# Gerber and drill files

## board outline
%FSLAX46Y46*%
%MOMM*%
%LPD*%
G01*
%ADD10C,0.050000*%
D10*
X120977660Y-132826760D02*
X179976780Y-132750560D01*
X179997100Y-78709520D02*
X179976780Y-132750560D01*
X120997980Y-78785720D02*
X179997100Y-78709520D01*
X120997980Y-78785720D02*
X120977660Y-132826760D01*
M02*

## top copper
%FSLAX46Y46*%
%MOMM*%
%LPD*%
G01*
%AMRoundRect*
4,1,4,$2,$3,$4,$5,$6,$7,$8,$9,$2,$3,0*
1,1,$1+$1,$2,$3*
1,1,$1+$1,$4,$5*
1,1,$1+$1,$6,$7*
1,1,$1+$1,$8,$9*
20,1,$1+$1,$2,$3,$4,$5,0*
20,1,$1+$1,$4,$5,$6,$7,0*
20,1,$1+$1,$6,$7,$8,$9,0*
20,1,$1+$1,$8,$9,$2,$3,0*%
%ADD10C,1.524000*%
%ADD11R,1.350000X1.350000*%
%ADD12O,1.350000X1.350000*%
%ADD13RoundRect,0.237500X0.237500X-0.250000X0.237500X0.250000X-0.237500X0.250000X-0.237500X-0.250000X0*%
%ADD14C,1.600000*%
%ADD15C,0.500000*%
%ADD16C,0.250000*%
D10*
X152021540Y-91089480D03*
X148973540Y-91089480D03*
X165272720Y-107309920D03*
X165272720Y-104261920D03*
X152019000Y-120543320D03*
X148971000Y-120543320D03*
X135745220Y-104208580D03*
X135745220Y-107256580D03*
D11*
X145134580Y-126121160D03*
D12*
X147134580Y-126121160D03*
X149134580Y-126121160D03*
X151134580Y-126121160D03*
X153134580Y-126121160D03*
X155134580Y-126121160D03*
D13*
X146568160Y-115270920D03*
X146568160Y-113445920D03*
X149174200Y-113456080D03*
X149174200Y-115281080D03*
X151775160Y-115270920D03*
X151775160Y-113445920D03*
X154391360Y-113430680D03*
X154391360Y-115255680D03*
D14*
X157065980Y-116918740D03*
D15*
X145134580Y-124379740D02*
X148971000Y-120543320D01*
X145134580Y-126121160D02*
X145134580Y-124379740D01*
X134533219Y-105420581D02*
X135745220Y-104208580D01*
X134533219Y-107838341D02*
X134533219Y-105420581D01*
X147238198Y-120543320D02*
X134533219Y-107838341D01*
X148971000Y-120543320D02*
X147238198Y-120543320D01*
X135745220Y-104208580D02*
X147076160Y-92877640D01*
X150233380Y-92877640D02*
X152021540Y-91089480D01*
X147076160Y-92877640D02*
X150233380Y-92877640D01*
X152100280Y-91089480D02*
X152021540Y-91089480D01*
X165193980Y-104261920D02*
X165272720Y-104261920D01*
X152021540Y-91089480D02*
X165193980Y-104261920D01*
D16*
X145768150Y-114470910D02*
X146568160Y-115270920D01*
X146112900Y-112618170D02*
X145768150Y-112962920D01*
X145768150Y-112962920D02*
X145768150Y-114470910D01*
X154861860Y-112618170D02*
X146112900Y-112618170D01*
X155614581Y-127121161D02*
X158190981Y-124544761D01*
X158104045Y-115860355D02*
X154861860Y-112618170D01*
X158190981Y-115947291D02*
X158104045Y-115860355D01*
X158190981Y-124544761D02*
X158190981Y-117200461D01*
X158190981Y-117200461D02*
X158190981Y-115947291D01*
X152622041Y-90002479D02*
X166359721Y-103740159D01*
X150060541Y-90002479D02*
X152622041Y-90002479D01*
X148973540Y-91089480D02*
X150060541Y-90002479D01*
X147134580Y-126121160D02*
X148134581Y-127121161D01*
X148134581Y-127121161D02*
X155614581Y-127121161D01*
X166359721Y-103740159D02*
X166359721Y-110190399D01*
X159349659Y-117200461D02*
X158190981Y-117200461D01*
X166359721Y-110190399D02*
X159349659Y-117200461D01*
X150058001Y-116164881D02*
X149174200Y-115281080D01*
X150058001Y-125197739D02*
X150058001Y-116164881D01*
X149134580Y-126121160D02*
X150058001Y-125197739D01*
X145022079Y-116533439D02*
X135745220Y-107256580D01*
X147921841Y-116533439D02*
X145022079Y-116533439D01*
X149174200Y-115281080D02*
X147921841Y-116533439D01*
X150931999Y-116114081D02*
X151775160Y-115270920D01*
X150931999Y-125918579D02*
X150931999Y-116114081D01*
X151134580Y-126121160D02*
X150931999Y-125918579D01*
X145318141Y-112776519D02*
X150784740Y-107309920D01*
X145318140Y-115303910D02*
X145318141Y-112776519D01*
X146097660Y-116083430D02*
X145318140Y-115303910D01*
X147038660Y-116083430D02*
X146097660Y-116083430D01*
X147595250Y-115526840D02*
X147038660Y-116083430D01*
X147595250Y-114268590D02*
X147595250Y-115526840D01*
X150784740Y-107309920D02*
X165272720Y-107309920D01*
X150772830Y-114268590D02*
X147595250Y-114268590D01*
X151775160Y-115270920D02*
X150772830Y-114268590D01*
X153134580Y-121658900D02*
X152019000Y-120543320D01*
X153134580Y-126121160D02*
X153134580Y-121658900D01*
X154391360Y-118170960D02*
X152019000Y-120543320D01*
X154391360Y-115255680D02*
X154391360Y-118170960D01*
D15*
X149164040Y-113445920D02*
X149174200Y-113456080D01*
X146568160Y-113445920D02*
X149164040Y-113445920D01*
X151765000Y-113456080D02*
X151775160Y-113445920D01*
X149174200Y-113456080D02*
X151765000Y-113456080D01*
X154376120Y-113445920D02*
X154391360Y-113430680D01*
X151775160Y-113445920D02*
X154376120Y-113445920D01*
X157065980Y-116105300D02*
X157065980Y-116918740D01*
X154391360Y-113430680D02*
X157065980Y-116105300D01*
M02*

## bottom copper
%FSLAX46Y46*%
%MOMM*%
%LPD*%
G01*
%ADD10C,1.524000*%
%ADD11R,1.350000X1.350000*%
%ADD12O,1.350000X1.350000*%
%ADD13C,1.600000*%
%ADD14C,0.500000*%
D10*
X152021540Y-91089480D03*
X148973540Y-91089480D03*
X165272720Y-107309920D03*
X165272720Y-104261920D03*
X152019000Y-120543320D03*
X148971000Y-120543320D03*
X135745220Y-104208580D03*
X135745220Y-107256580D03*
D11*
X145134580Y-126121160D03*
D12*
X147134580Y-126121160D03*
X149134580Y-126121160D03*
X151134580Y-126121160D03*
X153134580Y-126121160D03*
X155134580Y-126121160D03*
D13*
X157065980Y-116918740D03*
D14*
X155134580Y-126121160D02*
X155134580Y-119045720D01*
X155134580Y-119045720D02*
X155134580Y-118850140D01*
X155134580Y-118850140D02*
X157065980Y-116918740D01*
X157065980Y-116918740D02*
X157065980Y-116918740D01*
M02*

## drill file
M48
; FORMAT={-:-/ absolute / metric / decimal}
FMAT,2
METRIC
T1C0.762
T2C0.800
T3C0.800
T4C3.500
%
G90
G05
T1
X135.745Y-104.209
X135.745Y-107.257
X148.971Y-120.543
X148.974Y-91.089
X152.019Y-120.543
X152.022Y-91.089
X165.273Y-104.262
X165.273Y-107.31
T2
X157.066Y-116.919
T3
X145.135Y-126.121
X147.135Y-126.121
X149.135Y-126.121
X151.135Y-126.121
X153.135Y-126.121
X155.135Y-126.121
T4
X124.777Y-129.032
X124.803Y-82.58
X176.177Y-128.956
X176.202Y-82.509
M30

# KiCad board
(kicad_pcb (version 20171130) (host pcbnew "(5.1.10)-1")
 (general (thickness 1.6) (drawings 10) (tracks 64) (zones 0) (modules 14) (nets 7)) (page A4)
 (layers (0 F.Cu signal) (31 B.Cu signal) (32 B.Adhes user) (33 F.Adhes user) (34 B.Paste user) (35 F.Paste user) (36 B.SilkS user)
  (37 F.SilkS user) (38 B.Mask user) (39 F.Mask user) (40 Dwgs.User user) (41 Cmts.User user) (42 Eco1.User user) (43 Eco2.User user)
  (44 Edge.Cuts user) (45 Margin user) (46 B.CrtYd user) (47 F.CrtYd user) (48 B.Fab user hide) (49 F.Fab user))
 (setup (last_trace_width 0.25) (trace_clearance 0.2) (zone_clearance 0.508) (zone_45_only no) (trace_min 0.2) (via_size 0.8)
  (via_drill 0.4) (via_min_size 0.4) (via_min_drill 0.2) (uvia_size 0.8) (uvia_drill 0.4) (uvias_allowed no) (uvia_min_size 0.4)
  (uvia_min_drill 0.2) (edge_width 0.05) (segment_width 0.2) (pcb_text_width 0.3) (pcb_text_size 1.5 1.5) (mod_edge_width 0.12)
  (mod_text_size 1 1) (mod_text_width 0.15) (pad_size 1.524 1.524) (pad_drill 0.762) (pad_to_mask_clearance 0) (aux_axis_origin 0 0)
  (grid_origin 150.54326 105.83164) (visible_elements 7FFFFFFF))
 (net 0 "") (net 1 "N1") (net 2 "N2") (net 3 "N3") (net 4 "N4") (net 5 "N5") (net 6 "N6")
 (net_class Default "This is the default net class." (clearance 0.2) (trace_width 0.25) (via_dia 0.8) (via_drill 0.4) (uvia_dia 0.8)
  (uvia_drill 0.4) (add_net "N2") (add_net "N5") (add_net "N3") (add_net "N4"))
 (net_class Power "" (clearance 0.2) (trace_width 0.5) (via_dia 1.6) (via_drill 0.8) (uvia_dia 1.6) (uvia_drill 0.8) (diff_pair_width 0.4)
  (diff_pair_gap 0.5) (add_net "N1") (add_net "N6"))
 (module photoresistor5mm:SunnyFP (layer B.Cu) (at 150.43912 105.8418)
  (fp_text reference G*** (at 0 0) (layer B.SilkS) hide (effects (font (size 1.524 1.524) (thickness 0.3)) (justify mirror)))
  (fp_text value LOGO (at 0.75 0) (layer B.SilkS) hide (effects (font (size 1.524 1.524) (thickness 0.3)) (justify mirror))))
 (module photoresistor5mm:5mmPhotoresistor (layer F.Cu) (at 150.49754 91.08948 180)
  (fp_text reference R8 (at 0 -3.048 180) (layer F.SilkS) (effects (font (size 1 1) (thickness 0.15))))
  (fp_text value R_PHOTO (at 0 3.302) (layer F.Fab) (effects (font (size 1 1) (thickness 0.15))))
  (pad 1 thru_hole circle (at -1.524 0 180) (size 1.524 1.524) (drill 0.762) (layers *.Cu *.Mask) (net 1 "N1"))
  (pad 2 thru_hole circle (at 1.524 0 180) (size 1.524 1.524) (drill 0.762) (layers *.Cu *.Mask) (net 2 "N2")))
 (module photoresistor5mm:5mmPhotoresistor (layer F.Cu) (at 165.27272 105.78592 270)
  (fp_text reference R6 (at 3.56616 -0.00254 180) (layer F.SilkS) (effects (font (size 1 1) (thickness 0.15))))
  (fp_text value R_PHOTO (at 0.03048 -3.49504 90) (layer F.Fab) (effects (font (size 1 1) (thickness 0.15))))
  (pad 2 thru_hole circle (at 1.524 0 270) (size 1.524 1.524) (drill 0.762) (layers *.Cu *.Mask) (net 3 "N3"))
  (pad 1 thru_hole circle (at -1.524 0 270) (size 1.524 1.524) (drill 0.762) (layers *.Cu *.Mask) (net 1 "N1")))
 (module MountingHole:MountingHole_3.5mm (layer F.Cu) (at 176.17694 128.9558)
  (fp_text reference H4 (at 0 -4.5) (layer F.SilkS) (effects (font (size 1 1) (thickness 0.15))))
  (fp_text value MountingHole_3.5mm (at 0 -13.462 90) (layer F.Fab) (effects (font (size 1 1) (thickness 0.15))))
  (pad 1 np_thru_hole circle (at 0 0) (size 3.5 3.5) (drill 3.5) (layers *.Cu *.Mask)))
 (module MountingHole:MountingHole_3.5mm (layer F.Cu) (at 124.7775 129.032)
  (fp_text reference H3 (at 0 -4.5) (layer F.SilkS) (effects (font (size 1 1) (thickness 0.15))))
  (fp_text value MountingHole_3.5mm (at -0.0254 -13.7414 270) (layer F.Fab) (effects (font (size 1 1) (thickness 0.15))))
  (pad 1 np_thru_hole circle (at 0 0) (size 3.5 3.5) (drill 3.5) (layers *.Cu *.Mask)))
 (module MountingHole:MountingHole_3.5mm (layer F.Cu) (at 176.20234 82.50936 180)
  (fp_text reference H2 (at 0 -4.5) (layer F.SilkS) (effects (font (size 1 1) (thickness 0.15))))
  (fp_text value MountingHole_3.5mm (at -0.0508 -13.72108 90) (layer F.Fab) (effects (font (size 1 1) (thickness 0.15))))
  (pad 1 np_thru_hole circle (at 0 0 180) (size 3.5 3.5) (drill 3.5) (layers *.Cu *.Mask)))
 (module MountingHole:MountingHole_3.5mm (layer F.Cu) (at 124.8029 82.58048 180)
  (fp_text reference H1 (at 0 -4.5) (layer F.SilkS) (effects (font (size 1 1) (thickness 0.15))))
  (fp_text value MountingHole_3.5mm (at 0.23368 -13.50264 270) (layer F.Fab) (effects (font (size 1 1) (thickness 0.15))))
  (pad 1 np_thru_hole circle (at 0 0 180) (size 3.5 3.5) (drill 3.5) (layers *.Cu *.Mask)))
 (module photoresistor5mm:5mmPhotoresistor (layer F.Cu) (at 150.495 120.54332)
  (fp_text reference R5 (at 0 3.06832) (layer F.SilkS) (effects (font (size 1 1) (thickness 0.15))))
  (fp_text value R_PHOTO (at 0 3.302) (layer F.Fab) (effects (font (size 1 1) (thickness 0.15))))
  (pad 2 thru_hole circle (at 1.524 0) (size 1.524 1.524) (drill 0.762) (layers *.Cu *.Mask) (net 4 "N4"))
  (pad 1 thru_hole circle (at -1.524 0) (size 1.524 1.524) (drill 0.762) (layers *.Cu *.Mask) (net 1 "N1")))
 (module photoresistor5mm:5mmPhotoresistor (layer F.Cu) (at 135.74522 105.73258 270)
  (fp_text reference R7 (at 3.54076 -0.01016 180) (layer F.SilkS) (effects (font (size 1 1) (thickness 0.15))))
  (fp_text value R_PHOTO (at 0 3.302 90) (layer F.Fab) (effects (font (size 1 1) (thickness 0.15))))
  (pad 1 thru_hole circle (at -1.524 0 270) (size 1.524 1.524) (drill 0.762) (layers *.Cu *.Mask) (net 1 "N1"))
  (pad 2 thru_hole circle (at 1.524 0 270) (size 1.524 1.524) (drill 0.762) (layers *.Cu *.Mask) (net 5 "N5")))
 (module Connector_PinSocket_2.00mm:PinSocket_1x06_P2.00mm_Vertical (layer B.Cu) (at 145.13458 126.12116 270)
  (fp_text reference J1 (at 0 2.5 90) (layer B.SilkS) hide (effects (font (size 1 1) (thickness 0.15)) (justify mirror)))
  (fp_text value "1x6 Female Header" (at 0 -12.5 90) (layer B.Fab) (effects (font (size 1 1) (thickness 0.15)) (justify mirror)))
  (pad 1 thru_hole rect (at 0 0 270) (size 1.35 1.35) (drill 0.8) (layers *.Cu *.Mask) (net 1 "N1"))
  (pad 2 thru_hole oval (at 0 -2 270) (size 1.35 1.35) (drill 0.8) (layers *.Cu *.Mask) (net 2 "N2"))
  (pad 3 thru_hole oval (at 0 -4 270) (size 1.35 1.35) (drill 0.8) (layers *.Cu *.Mask) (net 5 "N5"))
  (pad 4 thru_hole oval (at 0 -6 270) (size 1.35 1.35) (drill 0.8) (layers *.Cu *.Mask) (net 3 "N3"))
  (pad 5 thru_hole oval (at 0 -8 270) (size 1.35 1.35) (drill 0.8) (layers *.Cu *.Mask) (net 4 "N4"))
  (pad 6 thru_hole oval (at 0 -10 270) (size 1.35 1.35) (drill 0.8) (layers *.Cu *.Mask) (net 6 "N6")))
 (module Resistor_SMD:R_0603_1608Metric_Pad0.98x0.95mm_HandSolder (layer F.Cu) (at 146.56816 114.35842 90)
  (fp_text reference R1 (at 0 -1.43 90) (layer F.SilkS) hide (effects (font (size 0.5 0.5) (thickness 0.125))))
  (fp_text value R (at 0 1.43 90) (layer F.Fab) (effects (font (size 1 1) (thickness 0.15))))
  (pad 1 smd roundrect (at -0.9125 0 90) (size 0.975 0.95) (layers F.Cu F.Paste F.Mask) (roundrect_rratio 0.25) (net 2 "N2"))
  (pad 2 smd roundrect (at 0.9125 0 90) (size 0.975 0.95) (layers F.Cu F.Paste F.Mask) (roundrect_rratio 0.25) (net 6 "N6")))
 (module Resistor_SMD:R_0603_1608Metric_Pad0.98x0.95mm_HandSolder (layer F.Cu) (at 149.1742 114.36858 90)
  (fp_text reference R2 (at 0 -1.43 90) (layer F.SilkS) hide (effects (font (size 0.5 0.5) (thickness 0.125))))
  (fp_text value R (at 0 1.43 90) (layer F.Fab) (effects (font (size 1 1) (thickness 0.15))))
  (pad 2 smd roundrect (at 0.9125 0 90) (size 0.975 0.95) (layers F.Cu F.Paste F.Mask) (roundrect_rratio 0.25) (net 6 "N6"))
  (pad 1 smd roundrect (at -0.9125 0 90) (size 0.975 0.95) (layers F.Cu F.Paste F.Mask) (roundrect_rratio 0.25) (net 5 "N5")))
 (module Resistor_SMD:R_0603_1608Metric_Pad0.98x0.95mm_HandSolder (layer F.Cu) (at 151.77516 114.35842 90)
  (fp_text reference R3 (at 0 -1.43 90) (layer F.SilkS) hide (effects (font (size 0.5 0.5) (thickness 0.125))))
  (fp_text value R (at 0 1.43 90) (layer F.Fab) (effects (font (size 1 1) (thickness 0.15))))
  (pad 1 smd roundrect (at -0.9125 0 90) (size 0.975 0.95) (layers F.Cu F.Paste F.Mask) (roundrect_rratio 0.25) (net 3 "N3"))
  (pad 2 smd roundrect (at 0.9125 0 90) (size 0.975 0.95) (layers F.Cu F.Paste F.Mask) (roundrect_rratio 0.25) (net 6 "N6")))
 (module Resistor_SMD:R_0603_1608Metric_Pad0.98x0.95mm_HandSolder (layer F.Cu) (at 154.39136 114.34318 90)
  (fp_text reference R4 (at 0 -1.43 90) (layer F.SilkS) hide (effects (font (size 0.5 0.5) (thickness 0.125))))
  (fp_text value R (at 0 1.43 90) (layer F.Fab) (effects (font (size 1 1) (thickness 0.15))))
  (pad 2 smd roundrect (at 0.9125 0 90) (size 0.975 0.95) (layers F.Cu F.Paste F.Mask) (roundrect_rratio 0.25) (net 6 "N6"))
  (pad 1 smd roundrect (at -0.9125 0 90) (size 0.975 0.95) (layers F.Cu F.Paste F.Mask) (roundrect_rratio 0.25) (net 4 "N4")))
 (gr_line (start 120.97766 132.82676) (end 179.97678 132.75056) (layer Edge.Cuts) (width 0.05))
 (gr_line (start 179.9971 78.70952) (end 179.97678 132.75056) (layer Edge.Cuts) (width 0.05))
 (gr_line (start 120.99798 78.78572) (end 179.9971 78.70952) (layer Edge.Cuts) (width 0.05))
 (gr_line (start 120.99798 78.78572) (end 120.97766 132.82676) (layer Edge.Cuts) (width 0.05))
 (segment (start 145.13458 124.37974) (end 148.971 120.54332) (width 0.5) (layer F.Cu) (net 1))
 (segment (start 145.13458 126.12116) (end 145.13458 124.37974) (width 0.5) (layer F.Cu) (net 1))
 (segment (start 134.533219 105.420581) (end 135.74522 104.20858) (width 0.5) (layer F.Cu) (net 1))
 (segment (start 134.533219 107.838341) (end 134.533219 105.420581) (width 0.5) (layer F.Cu) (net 1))
 (segment (start 147.238198 120.54332) (end 134.533219 107.838341) (width 0.5) (layer F.Cu) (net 1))
 (segment (start 148.971 120.54332) (end 147.238198 120.54332) (width 0.5) (layer F.Cu) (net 1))
 (segment (start 135.74522 104.20858) (end 147.07616 92.87764) (width 0.5) (layer F.Cu) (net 1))
 (segment (start 150.23338 92.87764) (end 152.02154 91.08948) (width 0.5) (layer F.Cu) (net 1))
 (segment (start 147.07616 92.87764) (end 150.23338 92.87764) (width 0.5) (layer F.Cu) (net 1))
 (segment (start 152.10028 91.08948) (end 152.02154 91.08948) (width 0.5) (layer F.Cu) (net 1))
 (segment (start 165.19398 104.26192) (end 165.27272 104.26192) (width 0.5) (layer F.Cu) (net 1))
 (segment (start 152.02154 91.08948) (end 165.19398 104.26192) (width 0.5) (layer F.Cu) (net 1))
 (segment (start 145.76815 114.47091) (end 146.56816 115.27092) (width 0.25) (layer F.Cu) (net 2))
 (segment (start 146.1129 112.61817) (end 145.76815 112.96292) (width 0.25) (layer F.Cu) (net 2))
 (segment (start 145.76815 112.96292) (end 145.76815 114.47091) (width 0.25) (layer F.Cu) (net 2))
 (segment (start 154.86186 112.61817) (end 146.1129 112.61817) (width 0.25) (layer F.Cu) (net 2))
 (segment (start 155.614581 127.121161) (end 158.190981 124.544761) (width 0.25) (layer F.Cu) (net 2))
 (segment (start 158.104045 115.860355) (end 154.86186 112.61817) (width 0.25) (layer F.Cu) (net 2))
 (segment (start 158.190981 115.947291) (end 158.104045 115.860355) (width 0.25) (layer F.Cu) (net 2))
 (segment (start 158.190981 124.544761) (end 158.190981 117.200461) (width 0.25) (layer F.Cu) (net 2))
 (segment (start 158.190981 117.200461) (end 158.190981 115.947291) (width 0.25) (layer F.Cu) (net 2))
 (segment (start 152.622041 90.002479) (end 166.359721 103.740159) (width 0.25) (layer F.Cu) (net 2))
 (segment (start 150.060541 90.002479) (end 152.622041 90.002479) (width 0.25) (layer F.Cu) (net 2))
 (segment (start 148.97354 91.08948) (end 150.060541 90.002479) (width 0.25) (layer F.Cu) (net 2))
 (segment (start 147.13458 126.12116) (end 148.134581 127.121161) (width 0.25) (layer F.Cu) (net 2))
 (segment (start 148.134581 127.121161) (end 155.614581 127.121161) (width 0.25) (layer F.Cu) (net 2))
 (segment (start 166.359721 103.740159) (end 166.359721 110.190399) (width 0.25) (layer F.Cu) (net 2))
 (segment (start 159.349659 117.200461) (end 158.190981 117.200461) (width 0.25) (layer F.Cu) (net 2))
 (segment (start 166.359721 110.190399) (end 159.349659 117.200461) (width 0.25) (layer F.Cu) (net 2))
 (segment (start 150.058001 116.164881) (end 149.1742 115.28108) (width 0.25) (layer F.Cu) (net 5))
 (segment (start 150.058001 125.197739) (end 150.058001 116.164881) (width 0.25) (layer F.Cu) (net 5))
 (segment (start 149.13458 126.12116) (end 150.058001 125.197739) (width 0.25) (layer F.Cu) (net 5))
 (segment (start 145.022079 116.533439) (end 135.74522 107.25658) (width 0.25) (layer F.Cu) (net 5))
 (segment (start 147.921841 116.533439) (end 145.022079 116.533439) (width 0.25) (layer F.Cu) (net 5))
 (segment (start 149.1742 115.28108) (end 147.921841 116.533439) (width 0.25) (layer F.Cu) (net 5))
 (segment (start 150.931999 116.114081) (end 151.77516 115.27092) (width 0.25) (layer F.Cu) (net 3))
 (segment (start 150.931999 125.918579) (end 150.931999 116.114081) (width 0.25) (layer F.Cu) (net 3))
 (segment (start 151.13458 126.12116) (end 150.931999 125.918579) (width 0.25) (layer F.Cu) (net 3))
 (segment (start 145.318141 112.776519) (end 150.78474 107.30992) (width 0.25) (layer F.Cu) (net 3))
 (segment (start 145.31814 115.30391) (end 145.318141 112.776519) (width 0.25) (layer F.Cu) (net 3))
 (segment (start 146.09766 116.08343) (end 145.31814 115.30391) (width 0.25) (layer F.Cu) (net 3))
 (segment (start 147.03866 116.08343) (end 146.09766 116.08343) (width 0.25) (layer F.Cu) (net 3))
 (segment (start 147.59525 115.52684) (end 147.03866 116.08343) (width 0.25) (layer F.Cu) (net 3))
 (segment (start 147.59525 114.26859) (end 147.59525 115.52684) (width 0.25) (layer F.Cu) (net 3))
 (segment (start 150.78474 107.30992) (end 165.27272 107.30992) (width 0.25) (layer F.Cu) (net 3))
 (segment (start 150.77283 114.26859) (end 147.59525 114.26859) (width 0.25) (layer F.Cu) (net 3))
 (segment (start 151.77516 115.27092) (end 150.77283 114.26859) (width 0.25) (layer F.Cu) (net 3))
 (segment (start 153.13458 121.6589) (end 152.019 120.54332) (width 0.25) (layer F.Cu) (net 4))
 (segment (start 153.13458 126.12116) (end 153.13458 121.6589) (width 0.25) (layer F.Cu) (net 4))
 (segment (start 154.39136 118.17096) (end 152.019 120.54332) (width 0.25) (layer F.Cu) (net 4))
 (segment (start 154.39136 115.25568) (end 154.39136 118.17096) (width 0.25) (layer F.Cu) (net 4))
 (segment (start 149.16404 113.44592) (end 149.1742 113.45608) (width 0.5) (layer F.Cu) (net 6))
 (segment (start 146.56816 113.44592) (end 149.16404 113.44592) (width 0.5) (layer F.Cu) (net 6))
 (segment (start 151.765 113.45608) (end 151.77516 113.44592) (width 0.5) (layer F.Cu) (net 6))
 (segment (start 149.1742 113.45608) (end 151.765 113.45608) (width 0.5) (layer F.Cu) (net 6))
 (segment (start 154.37612 113.44592) (end 154.39136 113.43068) (width 0.5) (layer F.Cu) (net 6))
 (segment (start 151.77516 113.44592) (end 154.37612 113.44592) (width 0.5) (layer F.Cu) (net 6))
 (segment (start 155.13458 126.12116) (end 155.13458 119.04572) (width 0.5) (layer B.Cu) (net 6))
 (segment (start 155.13458 119.04572) (end 155.13458 118.85014) (width 0.5) (layer B.Cu) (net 6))
 (segment (start 155.13458 118.85014) (end 157.06598 116.91874) (width 0.5) (layer B.Cu) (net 6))
 (segment (start 157.06598 116.91874) (end 157.06598 116.91874) (width 0.5) (layer B.Cu) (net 6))
 (via (at 157.06598 116.91874) (size 1.6) (drill 0.8) (layers F.Cu B.Cu) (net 6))
 (segment (start 157.06598 116.1053) (end 157.06598 116.91874) (width 0.5) (layer F.Cu) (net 6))
 (segment (start 154.39136 113.43068) (end 157.06598 116.1053) (width 0.5) (layer F.Cu) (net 6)))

